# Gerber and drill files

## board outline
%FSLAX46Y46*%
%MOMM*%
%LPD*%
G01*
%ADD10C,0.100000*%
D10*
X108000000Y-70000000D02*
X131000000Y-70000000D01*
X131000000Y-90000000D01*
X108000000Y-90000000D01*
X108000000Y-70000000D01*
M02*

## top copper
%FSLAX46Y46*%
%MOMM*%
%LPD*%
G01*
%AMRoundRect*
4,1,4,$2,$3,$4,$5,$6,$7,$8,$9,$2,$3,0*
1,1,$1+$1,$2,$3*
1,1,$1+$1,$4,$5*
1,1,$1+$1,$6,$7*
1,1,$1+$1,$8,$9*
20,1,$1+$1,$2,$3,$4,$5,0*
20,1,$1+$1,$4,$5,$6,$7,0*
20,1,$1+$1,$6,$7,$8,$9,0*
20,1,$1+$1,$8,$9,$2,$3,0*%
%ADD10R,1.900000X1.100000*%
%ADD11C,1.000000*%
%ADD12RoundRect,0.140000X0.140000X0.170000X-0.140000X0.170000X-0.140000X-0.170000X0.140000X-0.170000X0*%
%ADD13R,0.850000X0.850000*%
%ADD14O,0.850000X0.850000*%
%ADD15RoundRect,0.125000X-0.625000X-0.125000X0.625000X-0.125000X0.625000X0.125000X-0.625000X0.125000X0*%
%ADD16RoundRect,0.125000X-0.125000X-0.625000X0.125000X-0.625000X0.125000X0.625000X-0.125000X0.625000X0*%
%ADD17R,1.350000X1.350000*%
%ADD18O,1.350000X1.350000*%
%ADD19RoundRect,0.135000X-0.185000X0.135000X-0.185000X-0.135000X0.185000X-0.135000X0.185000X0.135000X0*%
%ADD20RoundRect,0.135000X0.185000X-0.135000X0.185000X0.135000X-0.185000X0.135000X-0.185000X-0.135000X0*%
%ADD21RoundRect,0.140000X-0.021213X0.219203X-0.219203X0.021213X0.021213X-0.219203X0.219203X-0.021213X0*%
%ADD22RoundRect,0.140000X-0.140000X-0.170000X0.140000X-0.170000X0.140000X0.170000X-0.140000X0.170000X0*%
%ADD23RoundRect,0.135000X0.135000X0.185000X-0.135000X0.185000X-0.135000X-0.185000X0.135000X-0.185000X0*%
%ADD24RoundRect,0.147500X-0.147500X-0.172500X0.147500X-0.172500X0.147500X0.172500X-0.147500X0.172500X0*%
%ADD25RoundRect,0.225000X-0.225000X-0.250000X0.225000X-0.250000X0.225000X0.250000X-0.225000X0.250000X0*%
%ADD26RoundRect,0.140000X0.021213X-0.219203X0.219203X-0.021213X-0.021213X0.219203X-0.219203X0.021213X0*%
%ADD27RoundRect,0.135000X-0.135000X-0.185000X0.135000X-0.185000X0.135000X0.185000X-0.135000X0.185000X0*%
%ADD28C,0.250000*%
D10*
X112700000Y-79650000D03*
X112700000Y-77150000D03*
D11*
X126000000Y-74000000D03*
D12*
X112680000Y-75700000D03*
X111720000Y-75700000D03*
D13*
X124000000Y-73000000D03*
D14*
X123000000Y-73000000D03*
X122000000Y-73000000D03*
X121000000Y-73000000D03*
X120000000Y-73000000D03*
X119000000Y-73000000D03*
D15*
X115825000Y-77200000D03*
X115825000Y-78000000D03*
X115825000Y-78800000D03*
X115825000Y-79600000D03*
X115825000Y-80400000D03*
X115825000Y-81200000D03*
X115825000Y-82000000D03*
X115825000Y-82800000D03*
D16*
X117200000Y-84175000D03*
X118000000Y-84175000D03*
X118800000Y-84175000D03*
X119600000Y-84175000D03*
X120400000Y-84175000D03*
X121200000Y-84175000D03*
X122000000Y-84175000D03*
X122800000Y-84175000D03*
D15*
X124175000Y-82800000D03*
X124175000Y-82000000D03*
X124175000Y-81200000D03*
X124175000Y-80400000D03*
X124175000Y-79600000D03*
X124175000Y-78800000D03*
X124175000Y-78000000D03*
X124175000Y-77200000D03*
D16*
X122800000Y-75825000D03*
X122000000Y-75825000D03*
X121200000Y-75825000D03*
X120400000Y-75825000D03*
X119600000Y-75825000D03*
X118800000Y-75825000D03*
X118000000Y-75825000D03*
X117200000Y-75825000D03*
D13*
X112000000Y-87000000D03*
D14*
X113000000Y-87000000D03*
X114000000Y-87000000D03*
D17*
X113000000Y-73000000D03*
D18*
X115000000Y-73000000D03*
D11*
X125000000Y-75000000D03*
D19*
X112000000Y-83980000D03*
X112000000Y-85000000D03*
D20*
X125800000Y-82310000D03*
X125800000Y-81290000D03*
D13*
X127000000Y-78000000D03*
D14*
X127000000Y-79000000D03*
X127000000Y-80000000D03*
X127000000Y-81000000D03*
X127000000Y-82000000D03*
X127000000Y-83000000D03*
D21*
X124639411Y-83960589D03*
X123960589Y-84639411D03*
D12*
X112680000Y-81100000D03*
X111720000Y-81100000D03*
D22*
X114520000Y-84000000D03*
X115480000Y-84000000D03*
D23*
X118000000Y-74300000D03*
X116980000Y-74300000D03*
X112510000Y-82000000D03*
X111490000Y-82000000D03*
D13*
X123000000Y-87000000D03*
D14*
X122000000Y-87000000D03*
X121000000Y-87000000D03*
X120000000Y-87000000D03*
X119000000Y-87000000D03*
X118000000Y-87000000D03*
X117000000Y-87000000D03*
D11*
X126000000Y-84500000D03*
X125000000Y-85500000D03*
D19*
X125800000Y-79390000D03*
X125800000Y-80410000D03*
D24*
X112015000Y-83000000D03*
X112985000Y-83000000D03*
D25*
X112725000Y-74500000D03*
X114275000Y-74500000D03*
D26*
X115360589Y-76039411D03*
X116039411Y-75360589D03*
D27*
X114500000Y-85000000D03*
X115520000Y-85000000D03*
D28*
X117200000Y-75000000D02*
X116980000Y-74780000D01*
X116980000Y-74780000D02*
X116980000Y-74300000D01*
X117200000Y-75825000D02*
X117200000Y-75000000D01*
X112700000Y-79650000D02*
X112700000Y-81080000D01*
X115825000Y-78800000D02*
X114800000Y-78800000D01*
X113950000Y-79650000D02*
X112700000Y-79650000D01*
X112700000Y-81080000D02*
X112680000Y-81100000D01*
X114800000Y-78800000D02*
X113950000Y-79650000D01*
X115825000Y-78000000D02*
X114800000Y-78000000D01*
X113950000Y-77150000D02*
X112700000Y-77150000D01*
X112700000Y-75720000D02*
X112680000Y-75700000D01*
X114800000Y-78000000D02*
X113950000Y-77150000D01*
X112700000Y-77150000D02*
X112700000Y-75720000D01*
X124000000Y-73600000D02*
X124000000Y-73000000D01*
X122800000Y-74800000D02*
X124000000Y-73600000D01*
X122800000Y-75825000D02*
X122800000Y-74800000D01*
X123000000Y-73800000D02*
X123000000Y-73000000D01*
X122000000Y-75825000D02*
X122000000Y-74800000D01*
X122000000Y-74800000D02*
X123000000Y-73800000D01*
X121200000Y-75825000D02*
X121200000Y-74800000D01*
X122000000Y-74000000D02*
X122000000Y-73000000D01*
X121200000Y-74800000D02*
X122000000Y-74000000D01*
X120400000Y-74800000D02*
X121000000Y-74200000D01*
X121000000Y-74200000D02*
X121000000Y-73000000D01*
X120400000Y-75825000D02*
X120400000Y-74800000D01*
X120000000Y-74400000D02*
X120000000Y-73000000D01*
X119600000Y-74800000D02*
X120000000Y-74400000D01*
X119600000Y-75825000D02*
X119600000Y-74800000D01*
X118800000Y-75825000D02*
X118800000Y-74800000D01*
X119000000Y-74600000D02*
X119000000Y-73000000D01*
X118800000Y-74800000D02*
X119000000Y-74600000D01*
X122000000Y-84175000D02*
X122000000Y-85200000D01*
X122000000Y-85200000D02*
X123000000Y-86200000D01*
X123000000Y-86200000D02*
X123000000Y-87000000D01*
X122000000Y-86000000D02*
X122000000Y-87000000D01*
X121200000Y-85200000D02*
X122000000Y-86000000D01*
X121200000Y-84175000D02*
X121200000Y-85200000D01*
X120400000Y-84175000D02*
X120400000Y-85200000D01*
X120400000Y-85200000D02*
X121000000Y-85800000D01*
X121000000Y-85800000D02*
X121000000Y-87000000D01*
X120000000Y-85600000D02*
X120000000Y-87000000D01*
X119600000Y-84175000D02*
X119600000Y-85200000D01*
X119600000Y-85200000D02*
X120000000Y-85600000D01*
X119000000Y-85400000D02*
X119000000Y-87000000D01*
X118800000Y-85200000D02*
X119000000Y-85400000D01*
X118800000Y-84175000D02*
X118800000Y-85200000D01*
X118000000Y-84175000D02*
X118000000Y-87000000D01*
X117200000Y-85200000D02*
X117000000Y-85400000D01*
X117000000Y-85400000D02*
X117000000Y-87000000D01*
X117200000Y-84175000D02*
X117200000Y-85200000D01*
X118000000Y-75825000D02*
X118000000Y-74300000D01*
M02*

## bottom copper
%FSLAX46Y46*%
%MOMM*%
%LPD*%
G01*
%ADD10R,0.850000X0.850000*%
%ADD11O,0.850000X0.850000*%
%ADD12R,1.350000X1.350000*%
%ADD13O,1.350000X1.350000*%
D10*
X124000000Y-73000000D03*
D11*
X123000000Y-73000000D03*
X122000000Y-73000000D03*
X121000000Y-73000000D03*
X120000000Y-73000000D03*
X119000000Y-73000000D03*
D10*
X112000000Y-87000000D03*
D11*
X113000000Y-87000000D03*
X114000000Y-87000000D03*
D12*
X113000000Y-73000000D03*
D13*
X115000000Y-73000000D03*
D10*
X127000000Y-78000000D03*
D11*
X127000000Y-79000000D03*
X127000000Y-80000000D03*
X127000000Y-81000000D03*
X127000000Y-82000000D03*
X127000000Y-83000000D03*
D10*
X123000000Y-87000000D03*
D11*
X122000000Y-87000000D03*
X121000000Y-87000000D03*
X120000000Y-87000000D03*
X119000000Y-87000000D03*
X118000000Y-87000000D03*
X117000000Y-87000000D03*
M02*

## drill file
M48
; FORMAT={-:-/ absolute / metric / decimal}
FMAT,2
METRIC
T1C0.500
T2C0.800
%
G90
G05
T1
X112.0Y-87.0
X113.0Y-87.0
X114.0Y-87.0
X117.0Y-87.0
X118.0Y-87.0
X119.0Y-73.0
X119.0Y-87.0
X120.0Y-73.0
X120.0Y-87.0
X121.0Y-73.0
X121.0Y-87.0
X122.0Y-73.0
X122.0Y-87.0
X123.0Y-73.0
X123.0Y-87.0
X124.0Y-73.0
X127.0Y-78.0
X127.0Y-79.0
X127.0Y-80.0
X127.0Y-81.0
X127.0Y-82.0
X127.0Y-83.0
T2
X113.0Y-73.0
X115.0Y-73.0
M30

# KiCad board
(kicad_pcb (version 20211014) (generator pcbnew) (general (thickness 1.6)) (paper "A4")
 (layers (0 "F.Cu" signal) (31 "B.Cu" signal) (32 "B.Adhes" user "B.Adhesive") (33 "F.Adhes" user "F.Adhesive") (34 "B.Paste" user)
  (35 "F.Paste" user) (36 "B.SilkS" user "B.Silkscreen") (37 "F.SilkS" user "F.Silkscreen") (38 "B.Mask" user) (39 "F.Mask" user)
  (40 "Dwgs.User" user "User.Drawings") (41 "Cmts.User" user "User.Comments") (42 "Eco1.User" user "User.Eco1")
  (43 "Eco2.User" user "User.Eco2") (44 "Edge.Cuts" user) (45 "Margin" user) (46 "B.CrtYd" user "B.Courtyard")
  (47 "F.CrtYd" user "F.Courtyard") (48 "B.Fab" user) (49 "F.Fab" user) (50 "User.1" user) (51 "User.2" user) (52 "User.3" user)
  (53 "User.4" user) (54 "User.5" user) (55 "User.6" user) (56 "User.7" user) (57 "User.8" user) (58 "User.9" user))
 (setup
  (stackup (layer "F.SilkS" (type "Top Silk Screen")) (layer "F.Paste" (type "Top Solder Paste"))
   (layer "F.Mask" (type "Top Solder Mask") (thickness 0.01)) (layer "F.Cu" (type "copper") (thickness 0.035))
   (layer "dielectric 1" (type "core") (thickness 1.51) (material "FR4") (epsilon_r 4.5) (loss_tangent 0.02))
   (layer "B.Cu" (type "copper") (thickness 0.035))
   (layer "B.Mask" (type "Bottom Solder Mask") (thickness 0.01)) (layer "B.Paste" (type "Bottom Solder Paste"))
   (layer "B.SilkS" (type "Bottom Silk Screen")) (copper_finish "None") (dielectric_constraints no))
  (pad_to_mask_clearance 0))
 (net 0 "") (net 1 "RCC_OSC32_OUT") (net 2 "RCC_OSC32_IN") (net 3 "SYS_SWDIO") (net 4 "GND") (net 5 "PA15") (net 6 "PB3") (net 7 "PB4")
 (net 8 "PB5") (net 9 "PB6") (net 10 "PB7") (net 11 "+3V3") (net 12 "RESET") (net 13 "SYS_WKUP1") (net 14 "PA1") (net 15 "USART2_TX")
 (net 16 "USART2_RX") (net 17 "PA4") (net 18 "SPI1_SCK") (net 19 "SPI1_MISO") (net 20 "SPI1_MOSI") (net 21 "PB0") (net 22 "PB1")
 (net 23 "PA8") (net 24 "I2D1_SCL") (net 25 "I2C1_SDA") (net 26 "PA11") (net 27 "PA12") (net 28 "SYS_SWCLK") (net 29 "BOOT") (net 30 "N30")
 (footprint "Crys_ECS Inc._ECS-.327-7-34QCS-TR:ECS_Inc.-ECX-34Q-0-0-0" (layer "F.Cu") (at 112.7 78.4 90)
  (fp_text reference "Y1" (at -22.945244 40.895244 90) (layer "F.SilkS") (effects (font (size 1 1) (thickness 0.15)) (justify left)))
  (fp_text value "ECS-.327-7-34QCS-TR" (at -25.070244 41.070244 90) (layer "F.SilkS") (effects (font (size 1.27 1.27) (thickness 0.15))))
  (pad "1" smd rect (at -1.25 0 90) (size 1.1 1.9) (layers "F.Cu" "F.Paste" "F.Mask") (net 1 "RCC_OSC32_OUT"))
  (pad "2" smd rect (at 1.25 0 90) (size 1.1 1.9) (layers "F.Cu" "F.Paste" "F.Mask") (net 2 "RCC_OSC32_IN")))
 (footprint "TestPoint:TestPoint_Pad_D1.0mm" (layer "F.Cu") (at 126 74)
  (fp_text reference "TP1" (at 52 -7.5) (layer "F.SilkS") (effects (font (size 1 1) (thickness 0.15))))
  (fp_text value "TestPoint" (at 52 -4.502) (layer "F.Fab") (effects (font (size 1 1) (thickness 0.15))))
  (pad "1" smd circle locked (at 0 0) (size 1 1) (layers "F.Cu" "F.Mask") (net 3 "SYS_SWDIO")))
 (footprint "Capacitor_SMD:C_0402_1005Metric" (layer "F.Cu") (at 112.2 75.7 180)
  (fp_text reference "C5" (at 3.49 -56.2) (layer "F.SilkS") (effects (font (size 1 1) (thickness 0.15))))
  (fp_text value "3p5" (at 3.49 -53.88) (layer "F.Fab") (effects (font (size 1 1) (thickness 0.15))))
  (pad "1" smd roundrect locked (at -0.48 0 180) (size 0.56 0.62) (layers "F.Cu" "F.Paste" "F.Mask") (roundrect_rratio 0.25)
   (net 2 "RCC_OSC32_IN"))
  (pad "2" smd roundrect locked (at 0.48 0 180) (size 0.56 0.62) (layers "F.Cu" "F.Paste" "F.Mask") (roundrect_rratio 0.25) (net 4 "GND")))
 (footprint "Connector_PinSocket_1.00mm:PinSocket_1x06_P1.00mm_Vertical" (layer "F.Cu") (at 124 73 -90)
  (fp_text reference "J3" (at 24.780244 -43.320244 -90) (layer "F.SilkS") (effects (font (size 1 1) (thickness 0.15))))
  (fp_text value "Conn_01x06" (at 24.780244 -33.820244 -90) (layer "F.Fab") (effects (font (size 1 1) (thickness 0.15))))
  (pad "1" thru_hole rect locked (at 0 0 270) (size 0.85 0.85) (drill 0.5) (layers *.Cu *.Mask) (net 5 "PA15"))
  (pad "2" thru_hole oval locked (at 0 1 270) (size 0.85 0.85) (drill 0.5) (layers *.Cu *.Mask) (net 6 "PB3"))
  (pad "3" thru_hole oval locked (at 0 2 270) (size 0.85 0.85) (drill 0.5) (layers *.Cu *.Mask) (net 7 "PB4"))
  (pad "4" thru_hole oval locked (at 0 3 270) (size 0.85 0.85) (drill 0.5) (layers *.Cu *.Mask) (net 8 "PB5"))
  (pad "5" thru_hole oval locked (at 0 4 270) (size 0.85 0.85) (drill 0.5) (layers *.Cu *.Mask) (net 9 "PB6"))
  (pad "6" thru_hole oval locked (at 0 5 270) (size 0.85 0.85) (drill 0.5) (layers *.Cu *.Mask) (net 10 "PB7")))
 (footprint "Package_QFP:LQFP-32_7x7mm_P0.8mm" (layer "F.Cu") (at 120 80)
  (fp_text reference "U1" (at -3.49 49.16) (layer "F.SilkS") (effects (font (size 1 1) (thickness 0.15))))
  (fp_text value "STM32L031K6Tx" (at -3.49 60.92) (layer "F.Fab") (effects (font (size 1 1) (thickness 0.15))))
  (pad "1" smd roundrect locked (at -4.175 -2.8) (size 1.5 0.5) (layers "F.Cu" "F.Paste" "F.Mask") (roundrect_rratio 0.25) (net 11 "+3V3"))
  (pad "2" smd roundrect locked (at -4.175 -2) (size 1.5 0.5) (layers "F.Cu" "F.Paste" "F.Mask") (roundrect_rratio 0.25)
   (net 2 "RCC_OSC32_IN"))
  (pad "3" smd roundrect locked (at -4.175 -1.2) (size 1.5 0.5) (layers "F.Cu" "F.Paste" "F.Mask") (roundrect_rratio 0.25)
   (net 1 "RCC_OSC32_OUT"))
  (pad "4" smd roundrect locked (at -4.175 -0.4) (size 1.5 0.5) (layers "F.Cu" "F.Paste" "F.Mask") (roundrect_rratio 0.25) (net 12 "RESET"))
  (pad "5" smd roundrect locked (at -4.175 0.4) (size 1.5 0.5) (layers "F.Cu" "F.Paste" "F.Mask") (roundrect_rratio 0.25) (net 11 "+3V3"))
  (pad "6" smd roundrect locked (at -4.175 1.2) (size 1.5 0.5) (layers "F.Cu" "F.Paste" "F.Mask") (roundrect_rratio 0.25)
   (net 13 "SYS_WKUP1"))
  (pad "7" smd roundrect locked (at -4.175 2) (size 1.5 0.5) (layers "F.Cu" "F.Paste" "F.Mask") (roundrect_rratio 0.25) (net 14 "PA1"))
  (pad "8" smd roundrect locked (at -4.175 2.8) (size 1.5 0.5) (layers "F.Cu" "F.Paste" "F.Mask") (roundrect_rratio 0.25)
   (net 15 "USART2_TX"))
  (pad "9" smd roundrect locked (at -2.8 4.175) (size 0.5 1.5) (layers "F.Cu" "F.Paste" "F.Mask") (roundrect_rratio 0.25)
   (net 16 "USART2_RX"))
  (pad "10" smd roundrect locked (at -2 4.175) (size 0.5 1.5) (layers "F.Cu" "F.Paste" "F.Mask") (roundrect_rratio 0.25) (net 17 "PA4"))
  (pad "11" smd roundrect locked (at -1.2 4.175) (size 0.5 1.5) (layers "F.Cu" "F.Paste" "F.Mask") (roundrect_rratio 0.25)
   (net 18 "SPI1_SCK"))
  (pad "12" smd roundrect locked (at -0.4 4.175) (size 0.5 1.5) (layers "F.Cu" "F.Paste" "F.Mask") (roundrect_rratio 0.25)
   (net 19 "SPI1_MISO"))
  (pad "13" smd roundrect locked (at 0.4 4.175) (size 0.5 1.5) (layers "F.Cu" "F.Paste" "F.Mask") (roundrect_rratio 0.25)
   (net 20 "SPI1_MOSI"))
  (pad "14" smd roundrect locked (at 1.2 4.175) (size 0.5 1.5) (layers "F.Cu" "F.Paste" "F.Mask") (roundrect_rratio 0.25) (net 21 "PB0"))
  (pad "15" smd roundrect locked (at 2 4.175) (size 0.5 1.5) (layers "F.Cu" "F.Paste" "F.Mask") (roundrect_rratio 0.25) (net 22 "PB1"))
  (pad "16" smd roundrect locked (at 2.8 4.175) (size 0.5 1.5) (layers "F.Cu" "F.Paste" "F.Mask") (roundrect_rratio 0.25) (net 4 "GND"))
  (pad "17" smd roundrect locked (at 4.175 2.8) (size 1.5 0.5) (layers "F.Cu" "F.Paste" "F.Mask") (roundrect_rratio 0.25) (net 11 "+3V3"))
  (pad "18" smd roundrect locked (at 4.175 2) (size 1.5 0.5) (layers "F.Cu" "F.Paste" "F.Mask") (roundrect_rratio 0.25) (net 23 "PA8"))
  (pad "19" smd roundrect locked (at 4.175 1.2) (size 1.5 0.5) (layers "F.Cu" "F.Paste" "F.Mask") (roundrect_rratio 0.25)
   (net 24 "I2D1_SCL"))
  (pad "20" smd roundrect locked (at 4.175 0.4) (size 1.5 0.5) (layers "F.Cu" "F.Paste" "F.Mask") (roundrect_rratio 0.25)
   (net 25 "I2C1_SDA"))
  (pad "21" smd roundrect locked (at 4.175 -0.4) (size 1.5 0.5) (layers "F.Cu" "F.Paste" "F.Mask") (roundrect_rratio 0.25) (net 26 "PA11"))
  (pad "22" smd roundrect locked (at 4.175 -1.2) (size 1.5 0.5) (layers "F.Cu" "F.Paste" "F.Mask") (roundrect_rratio 0.25) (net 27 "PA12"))
  (pad "23" smd roundrect locked (at 4.175 -2) (size 1.5 0.5) (layers "F.Cu" "F.Paste" "F.Mask") (roundrect_rratio 0.25) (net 3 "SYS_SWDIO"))
  (pad "24" smd roundrect locked (at 4.175 -2.8) (size 1.5 0.5) (layers "F.Cu" "F.Paste" "F.Mask") (roundrect_rratio 0.25)
   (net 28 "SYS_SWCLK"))
  (pad "25" smd roundrect locked (at 2.8 -4.175) (size 0.5 1.5) (layers "F.Cu" "F.Paste" "F.Mask") (roundrect_rratio 0.25) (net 5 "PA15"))
  (pad "26" smd roundrect locked (at 2 -4.175) (size 0.5 1.5) (layers "F.Cu" "F.Paste" "F.Mask") (roundrect_rratio 0.25) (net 6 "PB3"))
  (pad "27" smd roundrect locked (at 1.2 -4.175) (size 0.5 1.5) (layers "F.Cu" "F.Paste" "F.Mask") (roundrect_rratio 0.25) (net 7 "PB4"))
  (pad "28" smd roundrect locked (at 0.4 -4.175) (size 0.5 1.5) (layers "F.Cu" "F.Paste" "F.Mask") (roundrect_rratio 0.25) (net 8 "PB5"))
  (pad "29" smd roundrect locked (at -0.4 -4.175) (size 0.5 1.5) (layers "F.Cu" "F.Paste" "F.Mask") (roundrect_rratio 0.25) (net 9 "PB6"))
  (pad "30" smd roundrect locked (at -1.2 -4.175) (size 0.5 1.5) (layers "F.Cu" "F.Paste" "F.Mask") (roundrect_rratio 0.25) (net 10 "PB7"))
  (pad "31" smd roundrect locked (at -2 -4.175) (size 0.5 1.5) (layers "F.Cu" "F.Paste" "F.Mask") (roundrect_rratio 0.25) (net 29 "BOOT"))
  (pad "32" smd roundrect locked (at -2.8 -4.175) (size 0.5 1.5) (layers "F.Cu" "F.Paste" "F.Mask") (roundrect_rratio 0.25) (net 4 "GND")))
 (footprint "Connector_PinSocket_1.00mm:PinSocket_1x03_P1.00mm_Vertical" (layer "F.Cu") (at 112 87 90)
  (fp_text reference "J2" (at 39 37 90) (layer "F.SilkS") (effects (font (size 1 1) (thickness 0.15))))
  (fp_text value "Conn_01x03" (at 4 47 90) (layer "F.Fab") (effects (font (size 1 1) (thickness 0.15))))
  (pad "1" thru_hole rect locked (at 0 0 90) (size 0.85 0.85) (drill 0.5) (layers *.Cu *.Mask) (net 13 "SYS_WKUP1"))
  (pad "2" thru_hole oval locked (at 0 1 90) (size 0.85 0.85) (drill 0.5) (layers *.Cu *.Mask) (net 14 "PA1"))
  (pad "3" thru_hole oval locked (at 0 2 90) (size 0.85 0.85) (drill 0.5) (layers *.Cu *.Mask) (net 15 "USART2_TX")))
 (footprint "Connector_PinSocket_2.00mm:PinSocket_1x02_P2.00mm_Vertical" (layer "F.Cu") (at 113 73 90)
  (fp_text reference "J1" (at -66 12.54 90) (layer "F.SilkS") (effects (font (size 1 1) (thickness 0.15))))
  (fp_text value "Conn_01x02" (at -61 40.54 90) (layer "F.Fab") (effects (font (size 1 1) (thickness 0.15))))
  (pad "1" thru_hole rect locked (at 0 0 90) (size 1.35 1.35) (drill 0.8) (layers *.Cu *.Mask) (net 11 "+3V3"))
  (pad "2" thru_hole oval locked (at 0 2 90) (size 1.35 1.35) (drill 0.8) (layers *.Cu *.Mask) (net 4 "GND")))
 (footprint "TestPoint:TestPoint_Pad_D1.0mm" (layer "F.Cu") (at 125 75)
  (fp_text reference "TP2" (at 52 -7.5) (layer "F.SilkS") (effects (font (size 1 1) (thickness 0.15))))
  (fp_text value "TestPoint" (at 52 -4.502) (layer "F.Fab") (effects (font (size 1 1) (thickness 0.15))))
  (pad "1" smd circle locked (at 0 0) (size 1 1) (layers "F.Cu" "F.Mask") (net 28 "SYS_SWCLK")))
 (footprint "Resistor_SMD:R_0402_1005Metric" (layer "F.Cu") (at 112 84.49 -90)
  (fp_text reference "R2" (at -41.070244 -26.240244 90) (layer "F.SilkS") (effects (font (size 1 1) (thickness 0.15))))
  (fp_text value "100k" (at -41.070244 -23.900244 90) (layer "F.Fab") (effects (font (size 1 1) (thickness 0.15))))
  (pad "1" smd roundrect locked (at -0.51 0 270) (size 0.54 0.64) (layers "F.Cu" "F.Paste" "F.Mask") (roundrect_rratio 0.25)
   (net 13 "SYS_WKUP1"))
  (pad "2" smd roundrect locked (at 0.51 0 270) (size 0.54 0.64) (layers "F.Cu" "F.Paste" "F.Mask") (roundrect_rratio 0.25) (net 4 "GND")))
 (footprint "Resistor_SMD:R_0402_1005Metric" (layer "F.Cu") (at 125.8 81.8 90)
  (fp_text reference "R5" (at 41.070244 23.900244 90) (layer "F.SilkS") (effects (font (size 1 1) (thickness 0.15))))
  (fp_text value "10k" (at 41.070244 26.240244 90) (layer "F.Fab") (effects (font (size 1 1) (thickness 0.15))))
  (pad "1" smd roundrect locked (at -0.51 0 90) (size 0.54 0.64) (layers "F.Cu" "F.Paste" "F.Mask") (roundrect_rratio 0.25) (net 11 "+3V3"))
  (pad "2" smd roundrect locked (at 0.51 0 90) (size 0.54 0.64) (layers "F.Cu" "F.Paste" "F.Mask") (roundrect_rratio 0.25)
   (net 24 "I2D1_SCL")))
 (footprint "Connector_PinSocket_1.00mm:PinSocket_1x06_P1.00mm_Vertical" (layer "F.Cu") (at 127 78)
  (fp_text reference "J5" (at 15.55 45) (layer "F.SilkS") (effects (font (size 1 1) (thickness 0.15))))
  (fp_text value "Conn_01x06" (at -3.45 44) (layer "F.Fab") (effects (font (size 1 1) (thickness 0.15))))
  (pad "1" thru_hole rect locked (at 0 0) (size 0.85 0.85) (drill 0.5) (layers *.Cu *.Mask) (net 27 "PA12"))
  (pad "2" thru_hole oval locked (at 0 1) (size 0.85 0.85) (drill 0.5) (layers *.Cu *.Mask) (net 26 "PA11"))
  (pad "3" thru_hole oval locked (at 0 2) (size 0.85 0.85) (drill 0.5) (layers *.Cu *.Mask) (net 25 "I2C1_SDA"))
  (pad "4" thru_hole oval locked (at 0 3) (size 0.85 0.85) (drill 0.5) (layers *.Cu *.Mask) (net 24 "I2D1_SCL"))
  (pad "5" thru_hole oval locked (at 0 4) (size 0.85 0.85) (drill 0.5) (layers *.Cu *.Mask) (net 23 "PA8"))
  (pad "6" thru_hole oval locked (at 0 5) (size 0.85 0.85) (drill 0.5) (layers *.Cu *.Mask) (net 12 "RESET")))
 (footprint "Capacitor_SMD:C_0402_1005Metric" (layer "F.Cu") (at 124.3 84.3 -135)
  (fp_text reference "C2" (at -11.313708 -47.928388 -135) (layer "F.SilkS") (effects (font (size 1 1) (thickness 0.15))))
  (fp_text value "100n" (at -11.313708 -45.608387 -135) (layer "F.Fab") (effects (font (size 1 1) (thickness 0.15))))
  (pad "1" smd roundrect locked (at -0.48 0 225) (size 0.56 0.62) (layers "F.Cu" "F.Paste" "F.Mask") (roundrect_rratio 0.25) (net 11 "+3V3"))
  (pad "2" smd roundrect locked (at 0.48 0 225) (size 0.56 0.62) (layers "F.Cu" "F.Paste" "F.Mask") (roundrect_rratio 0.25) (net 4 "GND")))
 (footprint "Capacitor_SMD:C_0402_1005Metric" (layer "F.Cu") (at 112.2 81.1 180)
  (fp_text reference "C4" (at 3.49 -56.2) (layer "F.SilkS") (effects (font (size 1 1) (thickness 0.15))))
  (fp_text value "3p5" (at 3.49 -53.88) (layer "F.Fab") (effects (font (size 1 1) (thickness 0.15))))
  (pad "1" smd roundrect locked (at -0.48 0 180) (size 0.56 0.62) (layers "F.Cu" "F.Paste" "F.Mask") (roundrect_rratio 0.25)
   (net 1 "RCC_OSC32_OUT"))
  (pad "2" smd roundrect locked (at 0.48 0 180) (size 0.56 0.62) (layers "F.Cu" "F.Paste" "F.Mask") (roundrect_rratio 0.25) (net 4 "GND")))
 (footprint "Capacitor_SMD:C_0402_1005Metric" (layer "F.Cu") (at 115 84)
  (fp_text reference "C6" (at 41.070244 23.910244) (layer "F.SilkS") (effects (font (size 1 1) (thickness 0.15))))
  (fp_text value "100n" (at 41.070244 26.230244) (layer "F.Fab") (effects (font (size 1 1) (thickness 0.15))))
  (pad "1" smd roundrect locked (at -0.48 0) (size 0.56 0.62) (layers "F.Cu" "F.Paste" "F.Mask") (roundrect_rratio 0.25) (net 12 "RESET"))
  (pad "2" smd roundrect locked (at 0.48 0) (size 0.56 0.62) (layers "F.Cu" "F.Paste" "F.Mask") (roundrect_rratio 0.25) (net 4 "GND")))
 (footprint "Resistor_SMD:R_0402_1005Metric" (layer "F.Cu") (at 117.49 74.3 180)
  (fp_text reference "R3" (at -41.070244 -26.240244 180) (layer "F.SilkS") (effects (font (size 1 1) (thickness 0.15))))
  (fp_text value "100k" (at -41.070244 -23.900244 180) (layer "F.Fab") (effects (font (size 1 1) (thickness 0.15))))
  (pad "1" smd roundrect locked (at -0.51 0 180) (size 0.54 0.64) (layers "F.Cu" "F.Paste" "F.Mask") (roundrect_rratio 0.25) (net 29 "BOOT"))
  (pad "2" smd roundrect locked (at 0.51 0 180) (size 0.54 0.64) (layers "F.Cu" "F.Paste" "F.Mask") (roundrect_rratio 0.25) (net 4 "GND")))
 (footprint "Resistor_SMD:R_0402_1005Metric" (layer "F.Cu") (at 112 82 180)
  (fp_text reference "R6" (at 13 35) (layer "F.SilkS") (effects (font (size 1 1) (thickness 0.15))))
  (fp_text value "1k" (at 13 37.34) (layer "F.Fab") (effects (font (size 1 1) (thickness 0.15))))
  (pad "1" smd roundrect locked (at -0.51 0 180) (size 0.54 0.64) (layers "F.Cu" "F.Paste" "F.Mask") (roundrect_rratio 0.25) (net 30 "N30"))
  (pad "2" smd roundrect locked (at 0.51 0 180) (size 0.54 0.64) (layers "F.Cu" "F.Paste" "F.Mask") (roundrect_rratio 0.25) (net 4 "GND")))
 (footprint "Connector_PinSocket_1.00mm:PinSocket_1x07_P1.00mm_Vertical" (layer "F.Cu") (at 123 87 -90)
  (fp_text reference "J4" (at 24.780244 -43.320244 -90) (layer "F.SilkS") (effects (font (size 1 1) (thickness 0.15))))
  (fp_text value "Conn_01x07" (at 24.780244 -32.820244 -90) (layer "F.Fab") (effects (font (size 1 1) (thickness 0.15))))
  (pad "1" thru_hole rect locked (at 0 0 270) (size 0.85 0.85) (drill 0.5) (layers *.Cu *.Mask) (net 22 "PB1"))
  (pad "2" thru_hole oval locked (at 0 1 270) (size 0.85 0.85) (drill 0.5) (layers *.Cu *.Mask) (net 21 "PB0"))
  (pad "3" thru_hole oval locked (at 0 2 270) (size 0.85 0.85) (drill 0.5) (layers *.Cu *.Mask) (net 20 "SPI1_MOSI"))
  (pad "4" thru_hole oval locked (at 0 3 270) (size 0.85 0.85) (drill 0.5) (layers *.Cu *.Mask) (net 19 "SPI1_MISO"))
  (pad "5" thru_hole oval locked (at 0 4 270) (size 0.85 0.85) (drill 0.5) (layers *.Cu *.Mask) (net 18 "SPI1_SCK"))
  (pad "6" thru_hole oval locked (at 0 5 270) (size 0.85 0.85) (drill 0.5) (layers *.Cu *.Mask) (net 17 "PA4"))
  (pad "7" thru_hole oval locked (at 0 6 270) (size 0.85 0.85) (drill 0.5) (layers *.Cu *.Mask) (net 16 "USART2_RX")))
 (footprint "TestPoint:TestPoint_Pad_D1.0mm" (layer "F.Cu") (at 126 84.5)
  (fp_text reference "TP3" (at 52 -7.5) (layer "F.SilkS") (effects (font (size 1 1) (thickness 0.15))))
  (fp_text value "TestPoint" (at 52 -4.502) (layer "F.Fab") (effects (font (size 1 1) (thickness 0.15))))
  (pad "1" smd circle locked (at 0 0) (size 1 1) (layers "F.Cu" "F.Mask") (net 12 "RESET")))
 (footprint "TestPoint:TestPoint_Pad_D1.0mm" (layer "F.Cu") (at 125 85.5)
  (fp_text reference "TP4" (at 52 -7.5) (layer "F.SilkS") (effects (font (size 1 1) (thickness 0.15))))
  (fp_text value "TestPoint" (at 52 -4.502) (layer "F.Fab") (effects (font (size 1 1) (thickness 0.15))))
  (pad "1" smd circle locked (at 0 0) (size 1 1) (layers "F.Cu" "F.Mask") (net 4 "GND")))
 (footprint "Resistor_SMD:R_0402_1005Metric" (layer "F.Cu") (at 125.8 79.9 -90)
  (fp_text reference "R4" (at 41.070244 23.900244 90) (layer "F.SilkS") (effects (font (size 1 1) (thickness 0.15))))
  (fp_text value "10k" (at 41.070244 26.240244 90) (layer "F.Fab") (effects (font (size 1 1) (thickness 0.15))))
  (pad "1" smd roundrect locked (at -0.51 0 270) (size 0.54 0.64) (layers "F.Cu" "F.Paste" "F.Mask") (roundrect_rratio 0.25) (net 11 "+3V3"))
  (pad "2" smd roundrect locked (at 0.51 0 270) (size 0.54 0.64) (layers "F.Cu" "F.Paste" "F.Mask") (roundrect_rratio 0.25)
   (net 25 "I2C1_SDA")))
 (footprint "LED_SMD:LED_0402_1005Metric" (layer "F.Cu") (at 112.5 83)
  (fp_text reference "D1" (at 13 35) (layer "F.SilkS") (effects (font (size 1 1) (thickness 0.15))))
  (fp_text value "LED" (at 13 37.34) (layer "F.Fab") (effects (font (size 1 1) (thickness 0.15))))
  (pad "1" smd roundrect locked (at -0.485 0) (size 0.59 0.64) (layers "F.Cu" "F.Paste" "F.Mask") (roundrect_rratio 0.25) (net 30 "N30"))
  (pad "2" smd roundrect locked (at 0.485 0) (size 0.59 0.64) (layers "F.Cu" "F.Paste" "F.Mask") (roundrect_rratio 0.25) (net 14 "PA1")))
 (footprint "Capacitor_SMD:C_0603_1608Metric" (layer "F.Cu") (at 113.5 74.5)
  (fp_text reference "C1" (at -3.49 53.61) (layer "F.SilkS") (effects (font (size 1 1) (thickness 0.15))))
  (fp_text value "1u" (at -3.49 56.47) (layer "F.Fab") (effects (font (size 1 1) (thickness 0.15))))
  (pad "1" smd roundrect locked (at -0.775 0) (size 0.9 0.95) (layers "F.Cu" "F.Paste" "F.Mask") (roundrect_rratio 0.25) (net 11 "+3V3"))
  (pad "2" smd roundrect locked (at 0.775 0) (size 0.9 0.95) (layers "F.Cu" "F.Paste" "F.Mask") (roundrect_rratio 0.25) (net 4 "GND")))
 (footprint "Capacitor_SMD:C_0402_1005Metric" (layer "F.Cu") (at 115.7 75.7 45)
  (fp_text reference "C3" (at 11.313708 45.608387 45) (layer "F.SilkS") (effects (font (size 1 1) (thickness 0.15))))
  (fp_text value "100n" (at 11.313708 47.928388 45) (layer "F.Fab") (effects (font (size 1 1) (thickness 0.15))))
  (pad "1" smd roundrect locked (at -0.48 0 45) (size 0.56 0.62) (layers "F.Cu" "F.Paste" "F.Mask") (roundrect_rratio 0.25) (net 11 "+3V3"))
  (pad "2" smd roundrect locked (at 0.48 0 45) (size 0.56 0.62) (layers "F.Cu" "F.Paste" "F.Mask") (roundrect_rratio 0.25) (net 4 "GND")))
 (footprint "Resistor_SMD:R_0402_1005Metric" (layer "F.Cu") (at 115.01 85)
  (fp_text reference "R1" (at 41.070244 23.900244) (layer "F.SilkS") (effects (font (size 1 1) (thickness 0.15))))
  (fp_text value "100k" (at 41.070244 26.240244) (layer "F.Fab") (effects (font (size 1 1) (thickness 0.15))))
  (pad "1" smd roundrect locked (at -0.51 0) (size 0.54 0.64) (layers "F.Cu" "F.Paste" "F.Mask") (roundrect_rratio 0.25) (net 11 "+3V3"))
  (pad "2" smd roundrect locked (at 0.51 0) (size 0.54 0.64) (layers "F.Cu" "F.Paste" "F.Mask") (roundrect_rratio 0.25) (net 12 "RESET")))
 (gr_rect (start 108 70) (end 131 90) (layer "Edge.Cuts") (width 0.1) (fill none))
 (segment (start 117.2 75) (end 116.98 74.78) (width 0.25) (layer "F.Cu") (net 4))
 (segment (start 116.98 74.78) (end 116.98 74.3) (width 0.25) (layer "F.Cu") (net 4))
 (segment (start 117.2 75.825) (end 117.2 75) (width 0.25) (layer "F.Cu") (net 4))
 (segment (start 112.7 79.65) (end 112.7 81.08) (width 0.25) (layer "F.Cu") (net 1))
 (segment (start 115.825 78.8) (end 114.8 78.8) (width 0.25) (layer "F.Cu") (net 1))
 (segment (start 113.95 79.65) (end 112.7 79.65) (width 0.25) (layer "F.Cu") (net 1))
 (segment (start 112.7 81.08) (end 112.68 81.1) (width 0.25) (layer "F.Cu") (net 1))
 (segment (start 114.8 78.8) (end 113.95 79.65) (width 0.25) (layer "F.Cu") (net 1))
 (segment (start 115.825 78) (end 114.8 78) (width 0.25) (layer "F.Cu") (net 2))
 (segment (start 113.95 77.15) (end 112.7 77.15) (width 0.25) (layer "F.Cu") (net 2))
 (segment (start 112.7 75.72) (end 112.68 75.7) (width 0.25) (layer "F.Cu") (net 2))
 (segment (start 114.8 78) (end 113.95 77.15) (width 0.25) (layer "F.Cu") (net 2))
 (segment (start 112.7 77.15) (end 112.7 75.72) (width 0.25) (layer "F.Cu") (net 2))
 (segment (start 124 73.6) (end 124 73) (width 0.25) (layer "F.Cu") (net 5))
 (segment (start 122.8 74.8) (end 124 73.6) (width 0.25) (layer "F.Cu") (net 5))
 (segment (start 122.8 75.825) (end 122.8 74.8) (width 0.25) (layer "F.Cu") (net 5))
 (segment (start 123 73.8) (end 123 73) (width 0.25) (layer "F.Cu") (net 6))
 (segment (start 122 75.825) (end 122 74.8) (width 0.25) (layer "F.Cu") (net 6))
 (segment (start 122 74.8) (end 123 73.8) (width 0.25) (layer "F.Cu") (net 6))
 (segment (start 121.2 75.825) (end 121.2 74.8) (width 0.25) (layer "F.Cu") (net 7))
 (segment (start 122 74) (end 122 73) (width 0.25) (layer "F.Cu") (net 7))
 (segment (start 121.2 74.8) (end 122 74) (width 0.25) (layer "F.Cu") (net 7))
 (segment (start 120.4 74.8) (end 121 74.2) (width 0.25) (layer "F.Cu") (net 8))
 (segment (start 121 74.2) (end 121 73) (width 0.25) (layer "F.Cu") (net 8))
 (segment (start 120.4 75.825) (end 120.4 74.8) (width 0.25) (layer "F.Cu") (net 8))
 (segment (start 120 74.4) (end 120 73) (width 0.25) (layer "F.Cu") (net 9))
 (segment (start 119.6 74.8) (end 120 74.4) (width 0.25) (layer "F.Cu") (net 9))
 (segment (start 119.6 75.825) (end 119.6 74.8) (width 0.25) (layer "F.Cu") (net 9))
 (segment (start 118.8 75.825) (end 118.8 74.8) (width 0.25) (layer "F.Cu") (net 10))
 (segment (start 119 74.6) (end 119 73) (width 0.25) (layer "F.Cu") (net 10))
 (segment (start 118.8 74.8) (end 119 74.6) (width 0.25) (layer "F.Cu") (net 10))
 (segment (start 122 84.175) (end 122 85.2) (width 0.25) (layer "F.Cu") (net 22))
 (segment (start 122 85.2) (end 123 86.2) (width 0.25) (layer "F.Cu") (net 22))
 (segment (start 123 86.2) (end 123 87) (width 0.25) (layer "F.Cu") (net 22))
 (segment (start 122 86) (end 122 87) (width 0.25) (layer "F.Cu") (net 21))
 (segment (start 121.2 85.2) (end 122 86) (width 0.25) (layer "F.Cu") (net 21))
 (segment (start 121.2 84.175) (end 121.2 85.2) (width 0.25) (layer "F.Cu") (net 21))
 (segment (start 120.4 84.175) (end 120.4 85.2) (width 0.25) (layer "F.Cu") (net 20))
 (segment (start 120.4 85.2) (end 121 85.8) (width 0.25) (layer "F.Cu") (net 20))
 (segment (start 121 85.8) (end 121 87) (width 0.25) (layer "F.Cu") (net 20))
 (segment (start 120 85.6) (end 120 87) (width 0.25) (layer "F.Cu") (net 19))
 (segment (start 119.6 84.175) (end 119.6 85.2) (width 0.25) (layer "F.Cu") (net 19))
 (segment (start 119.6 85.2) (end 120 85.6) (width 0.25) (layer "F.Cu") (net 19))
 (segment (start 119 85.4) (end 119 87) (width 0.25) (layer "F.Cu") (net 18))
 (segment (start 118.8 85.2) (end 119 85.4) (width 0.25) (layer "F.Cu") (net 18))
 (segment (start 118.8 84.175) (end 118.8 85.2) (width 0.25) (layer "F.Cu") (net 18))
 (segment (start 118 84.175) (end 118 87) (width 0.25) (layer "F.Cu") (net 17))
 (segment (start 117.2 85.2) (end 117 85.4) (width 0.25) (layer "F.Cu") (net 16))
 (segment (start 117 85.4) (end 117 87) (width 0.25) (layer "F.Cu") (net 16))
 (segment (start 117.2 84.175) (end 117.2 85.2) (width 0.25) (layer "F.Cu") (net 16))
 (segment (start 118 75.825) (end 118 74.3) (width 0.25) (layer "F.Cu") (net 29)))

